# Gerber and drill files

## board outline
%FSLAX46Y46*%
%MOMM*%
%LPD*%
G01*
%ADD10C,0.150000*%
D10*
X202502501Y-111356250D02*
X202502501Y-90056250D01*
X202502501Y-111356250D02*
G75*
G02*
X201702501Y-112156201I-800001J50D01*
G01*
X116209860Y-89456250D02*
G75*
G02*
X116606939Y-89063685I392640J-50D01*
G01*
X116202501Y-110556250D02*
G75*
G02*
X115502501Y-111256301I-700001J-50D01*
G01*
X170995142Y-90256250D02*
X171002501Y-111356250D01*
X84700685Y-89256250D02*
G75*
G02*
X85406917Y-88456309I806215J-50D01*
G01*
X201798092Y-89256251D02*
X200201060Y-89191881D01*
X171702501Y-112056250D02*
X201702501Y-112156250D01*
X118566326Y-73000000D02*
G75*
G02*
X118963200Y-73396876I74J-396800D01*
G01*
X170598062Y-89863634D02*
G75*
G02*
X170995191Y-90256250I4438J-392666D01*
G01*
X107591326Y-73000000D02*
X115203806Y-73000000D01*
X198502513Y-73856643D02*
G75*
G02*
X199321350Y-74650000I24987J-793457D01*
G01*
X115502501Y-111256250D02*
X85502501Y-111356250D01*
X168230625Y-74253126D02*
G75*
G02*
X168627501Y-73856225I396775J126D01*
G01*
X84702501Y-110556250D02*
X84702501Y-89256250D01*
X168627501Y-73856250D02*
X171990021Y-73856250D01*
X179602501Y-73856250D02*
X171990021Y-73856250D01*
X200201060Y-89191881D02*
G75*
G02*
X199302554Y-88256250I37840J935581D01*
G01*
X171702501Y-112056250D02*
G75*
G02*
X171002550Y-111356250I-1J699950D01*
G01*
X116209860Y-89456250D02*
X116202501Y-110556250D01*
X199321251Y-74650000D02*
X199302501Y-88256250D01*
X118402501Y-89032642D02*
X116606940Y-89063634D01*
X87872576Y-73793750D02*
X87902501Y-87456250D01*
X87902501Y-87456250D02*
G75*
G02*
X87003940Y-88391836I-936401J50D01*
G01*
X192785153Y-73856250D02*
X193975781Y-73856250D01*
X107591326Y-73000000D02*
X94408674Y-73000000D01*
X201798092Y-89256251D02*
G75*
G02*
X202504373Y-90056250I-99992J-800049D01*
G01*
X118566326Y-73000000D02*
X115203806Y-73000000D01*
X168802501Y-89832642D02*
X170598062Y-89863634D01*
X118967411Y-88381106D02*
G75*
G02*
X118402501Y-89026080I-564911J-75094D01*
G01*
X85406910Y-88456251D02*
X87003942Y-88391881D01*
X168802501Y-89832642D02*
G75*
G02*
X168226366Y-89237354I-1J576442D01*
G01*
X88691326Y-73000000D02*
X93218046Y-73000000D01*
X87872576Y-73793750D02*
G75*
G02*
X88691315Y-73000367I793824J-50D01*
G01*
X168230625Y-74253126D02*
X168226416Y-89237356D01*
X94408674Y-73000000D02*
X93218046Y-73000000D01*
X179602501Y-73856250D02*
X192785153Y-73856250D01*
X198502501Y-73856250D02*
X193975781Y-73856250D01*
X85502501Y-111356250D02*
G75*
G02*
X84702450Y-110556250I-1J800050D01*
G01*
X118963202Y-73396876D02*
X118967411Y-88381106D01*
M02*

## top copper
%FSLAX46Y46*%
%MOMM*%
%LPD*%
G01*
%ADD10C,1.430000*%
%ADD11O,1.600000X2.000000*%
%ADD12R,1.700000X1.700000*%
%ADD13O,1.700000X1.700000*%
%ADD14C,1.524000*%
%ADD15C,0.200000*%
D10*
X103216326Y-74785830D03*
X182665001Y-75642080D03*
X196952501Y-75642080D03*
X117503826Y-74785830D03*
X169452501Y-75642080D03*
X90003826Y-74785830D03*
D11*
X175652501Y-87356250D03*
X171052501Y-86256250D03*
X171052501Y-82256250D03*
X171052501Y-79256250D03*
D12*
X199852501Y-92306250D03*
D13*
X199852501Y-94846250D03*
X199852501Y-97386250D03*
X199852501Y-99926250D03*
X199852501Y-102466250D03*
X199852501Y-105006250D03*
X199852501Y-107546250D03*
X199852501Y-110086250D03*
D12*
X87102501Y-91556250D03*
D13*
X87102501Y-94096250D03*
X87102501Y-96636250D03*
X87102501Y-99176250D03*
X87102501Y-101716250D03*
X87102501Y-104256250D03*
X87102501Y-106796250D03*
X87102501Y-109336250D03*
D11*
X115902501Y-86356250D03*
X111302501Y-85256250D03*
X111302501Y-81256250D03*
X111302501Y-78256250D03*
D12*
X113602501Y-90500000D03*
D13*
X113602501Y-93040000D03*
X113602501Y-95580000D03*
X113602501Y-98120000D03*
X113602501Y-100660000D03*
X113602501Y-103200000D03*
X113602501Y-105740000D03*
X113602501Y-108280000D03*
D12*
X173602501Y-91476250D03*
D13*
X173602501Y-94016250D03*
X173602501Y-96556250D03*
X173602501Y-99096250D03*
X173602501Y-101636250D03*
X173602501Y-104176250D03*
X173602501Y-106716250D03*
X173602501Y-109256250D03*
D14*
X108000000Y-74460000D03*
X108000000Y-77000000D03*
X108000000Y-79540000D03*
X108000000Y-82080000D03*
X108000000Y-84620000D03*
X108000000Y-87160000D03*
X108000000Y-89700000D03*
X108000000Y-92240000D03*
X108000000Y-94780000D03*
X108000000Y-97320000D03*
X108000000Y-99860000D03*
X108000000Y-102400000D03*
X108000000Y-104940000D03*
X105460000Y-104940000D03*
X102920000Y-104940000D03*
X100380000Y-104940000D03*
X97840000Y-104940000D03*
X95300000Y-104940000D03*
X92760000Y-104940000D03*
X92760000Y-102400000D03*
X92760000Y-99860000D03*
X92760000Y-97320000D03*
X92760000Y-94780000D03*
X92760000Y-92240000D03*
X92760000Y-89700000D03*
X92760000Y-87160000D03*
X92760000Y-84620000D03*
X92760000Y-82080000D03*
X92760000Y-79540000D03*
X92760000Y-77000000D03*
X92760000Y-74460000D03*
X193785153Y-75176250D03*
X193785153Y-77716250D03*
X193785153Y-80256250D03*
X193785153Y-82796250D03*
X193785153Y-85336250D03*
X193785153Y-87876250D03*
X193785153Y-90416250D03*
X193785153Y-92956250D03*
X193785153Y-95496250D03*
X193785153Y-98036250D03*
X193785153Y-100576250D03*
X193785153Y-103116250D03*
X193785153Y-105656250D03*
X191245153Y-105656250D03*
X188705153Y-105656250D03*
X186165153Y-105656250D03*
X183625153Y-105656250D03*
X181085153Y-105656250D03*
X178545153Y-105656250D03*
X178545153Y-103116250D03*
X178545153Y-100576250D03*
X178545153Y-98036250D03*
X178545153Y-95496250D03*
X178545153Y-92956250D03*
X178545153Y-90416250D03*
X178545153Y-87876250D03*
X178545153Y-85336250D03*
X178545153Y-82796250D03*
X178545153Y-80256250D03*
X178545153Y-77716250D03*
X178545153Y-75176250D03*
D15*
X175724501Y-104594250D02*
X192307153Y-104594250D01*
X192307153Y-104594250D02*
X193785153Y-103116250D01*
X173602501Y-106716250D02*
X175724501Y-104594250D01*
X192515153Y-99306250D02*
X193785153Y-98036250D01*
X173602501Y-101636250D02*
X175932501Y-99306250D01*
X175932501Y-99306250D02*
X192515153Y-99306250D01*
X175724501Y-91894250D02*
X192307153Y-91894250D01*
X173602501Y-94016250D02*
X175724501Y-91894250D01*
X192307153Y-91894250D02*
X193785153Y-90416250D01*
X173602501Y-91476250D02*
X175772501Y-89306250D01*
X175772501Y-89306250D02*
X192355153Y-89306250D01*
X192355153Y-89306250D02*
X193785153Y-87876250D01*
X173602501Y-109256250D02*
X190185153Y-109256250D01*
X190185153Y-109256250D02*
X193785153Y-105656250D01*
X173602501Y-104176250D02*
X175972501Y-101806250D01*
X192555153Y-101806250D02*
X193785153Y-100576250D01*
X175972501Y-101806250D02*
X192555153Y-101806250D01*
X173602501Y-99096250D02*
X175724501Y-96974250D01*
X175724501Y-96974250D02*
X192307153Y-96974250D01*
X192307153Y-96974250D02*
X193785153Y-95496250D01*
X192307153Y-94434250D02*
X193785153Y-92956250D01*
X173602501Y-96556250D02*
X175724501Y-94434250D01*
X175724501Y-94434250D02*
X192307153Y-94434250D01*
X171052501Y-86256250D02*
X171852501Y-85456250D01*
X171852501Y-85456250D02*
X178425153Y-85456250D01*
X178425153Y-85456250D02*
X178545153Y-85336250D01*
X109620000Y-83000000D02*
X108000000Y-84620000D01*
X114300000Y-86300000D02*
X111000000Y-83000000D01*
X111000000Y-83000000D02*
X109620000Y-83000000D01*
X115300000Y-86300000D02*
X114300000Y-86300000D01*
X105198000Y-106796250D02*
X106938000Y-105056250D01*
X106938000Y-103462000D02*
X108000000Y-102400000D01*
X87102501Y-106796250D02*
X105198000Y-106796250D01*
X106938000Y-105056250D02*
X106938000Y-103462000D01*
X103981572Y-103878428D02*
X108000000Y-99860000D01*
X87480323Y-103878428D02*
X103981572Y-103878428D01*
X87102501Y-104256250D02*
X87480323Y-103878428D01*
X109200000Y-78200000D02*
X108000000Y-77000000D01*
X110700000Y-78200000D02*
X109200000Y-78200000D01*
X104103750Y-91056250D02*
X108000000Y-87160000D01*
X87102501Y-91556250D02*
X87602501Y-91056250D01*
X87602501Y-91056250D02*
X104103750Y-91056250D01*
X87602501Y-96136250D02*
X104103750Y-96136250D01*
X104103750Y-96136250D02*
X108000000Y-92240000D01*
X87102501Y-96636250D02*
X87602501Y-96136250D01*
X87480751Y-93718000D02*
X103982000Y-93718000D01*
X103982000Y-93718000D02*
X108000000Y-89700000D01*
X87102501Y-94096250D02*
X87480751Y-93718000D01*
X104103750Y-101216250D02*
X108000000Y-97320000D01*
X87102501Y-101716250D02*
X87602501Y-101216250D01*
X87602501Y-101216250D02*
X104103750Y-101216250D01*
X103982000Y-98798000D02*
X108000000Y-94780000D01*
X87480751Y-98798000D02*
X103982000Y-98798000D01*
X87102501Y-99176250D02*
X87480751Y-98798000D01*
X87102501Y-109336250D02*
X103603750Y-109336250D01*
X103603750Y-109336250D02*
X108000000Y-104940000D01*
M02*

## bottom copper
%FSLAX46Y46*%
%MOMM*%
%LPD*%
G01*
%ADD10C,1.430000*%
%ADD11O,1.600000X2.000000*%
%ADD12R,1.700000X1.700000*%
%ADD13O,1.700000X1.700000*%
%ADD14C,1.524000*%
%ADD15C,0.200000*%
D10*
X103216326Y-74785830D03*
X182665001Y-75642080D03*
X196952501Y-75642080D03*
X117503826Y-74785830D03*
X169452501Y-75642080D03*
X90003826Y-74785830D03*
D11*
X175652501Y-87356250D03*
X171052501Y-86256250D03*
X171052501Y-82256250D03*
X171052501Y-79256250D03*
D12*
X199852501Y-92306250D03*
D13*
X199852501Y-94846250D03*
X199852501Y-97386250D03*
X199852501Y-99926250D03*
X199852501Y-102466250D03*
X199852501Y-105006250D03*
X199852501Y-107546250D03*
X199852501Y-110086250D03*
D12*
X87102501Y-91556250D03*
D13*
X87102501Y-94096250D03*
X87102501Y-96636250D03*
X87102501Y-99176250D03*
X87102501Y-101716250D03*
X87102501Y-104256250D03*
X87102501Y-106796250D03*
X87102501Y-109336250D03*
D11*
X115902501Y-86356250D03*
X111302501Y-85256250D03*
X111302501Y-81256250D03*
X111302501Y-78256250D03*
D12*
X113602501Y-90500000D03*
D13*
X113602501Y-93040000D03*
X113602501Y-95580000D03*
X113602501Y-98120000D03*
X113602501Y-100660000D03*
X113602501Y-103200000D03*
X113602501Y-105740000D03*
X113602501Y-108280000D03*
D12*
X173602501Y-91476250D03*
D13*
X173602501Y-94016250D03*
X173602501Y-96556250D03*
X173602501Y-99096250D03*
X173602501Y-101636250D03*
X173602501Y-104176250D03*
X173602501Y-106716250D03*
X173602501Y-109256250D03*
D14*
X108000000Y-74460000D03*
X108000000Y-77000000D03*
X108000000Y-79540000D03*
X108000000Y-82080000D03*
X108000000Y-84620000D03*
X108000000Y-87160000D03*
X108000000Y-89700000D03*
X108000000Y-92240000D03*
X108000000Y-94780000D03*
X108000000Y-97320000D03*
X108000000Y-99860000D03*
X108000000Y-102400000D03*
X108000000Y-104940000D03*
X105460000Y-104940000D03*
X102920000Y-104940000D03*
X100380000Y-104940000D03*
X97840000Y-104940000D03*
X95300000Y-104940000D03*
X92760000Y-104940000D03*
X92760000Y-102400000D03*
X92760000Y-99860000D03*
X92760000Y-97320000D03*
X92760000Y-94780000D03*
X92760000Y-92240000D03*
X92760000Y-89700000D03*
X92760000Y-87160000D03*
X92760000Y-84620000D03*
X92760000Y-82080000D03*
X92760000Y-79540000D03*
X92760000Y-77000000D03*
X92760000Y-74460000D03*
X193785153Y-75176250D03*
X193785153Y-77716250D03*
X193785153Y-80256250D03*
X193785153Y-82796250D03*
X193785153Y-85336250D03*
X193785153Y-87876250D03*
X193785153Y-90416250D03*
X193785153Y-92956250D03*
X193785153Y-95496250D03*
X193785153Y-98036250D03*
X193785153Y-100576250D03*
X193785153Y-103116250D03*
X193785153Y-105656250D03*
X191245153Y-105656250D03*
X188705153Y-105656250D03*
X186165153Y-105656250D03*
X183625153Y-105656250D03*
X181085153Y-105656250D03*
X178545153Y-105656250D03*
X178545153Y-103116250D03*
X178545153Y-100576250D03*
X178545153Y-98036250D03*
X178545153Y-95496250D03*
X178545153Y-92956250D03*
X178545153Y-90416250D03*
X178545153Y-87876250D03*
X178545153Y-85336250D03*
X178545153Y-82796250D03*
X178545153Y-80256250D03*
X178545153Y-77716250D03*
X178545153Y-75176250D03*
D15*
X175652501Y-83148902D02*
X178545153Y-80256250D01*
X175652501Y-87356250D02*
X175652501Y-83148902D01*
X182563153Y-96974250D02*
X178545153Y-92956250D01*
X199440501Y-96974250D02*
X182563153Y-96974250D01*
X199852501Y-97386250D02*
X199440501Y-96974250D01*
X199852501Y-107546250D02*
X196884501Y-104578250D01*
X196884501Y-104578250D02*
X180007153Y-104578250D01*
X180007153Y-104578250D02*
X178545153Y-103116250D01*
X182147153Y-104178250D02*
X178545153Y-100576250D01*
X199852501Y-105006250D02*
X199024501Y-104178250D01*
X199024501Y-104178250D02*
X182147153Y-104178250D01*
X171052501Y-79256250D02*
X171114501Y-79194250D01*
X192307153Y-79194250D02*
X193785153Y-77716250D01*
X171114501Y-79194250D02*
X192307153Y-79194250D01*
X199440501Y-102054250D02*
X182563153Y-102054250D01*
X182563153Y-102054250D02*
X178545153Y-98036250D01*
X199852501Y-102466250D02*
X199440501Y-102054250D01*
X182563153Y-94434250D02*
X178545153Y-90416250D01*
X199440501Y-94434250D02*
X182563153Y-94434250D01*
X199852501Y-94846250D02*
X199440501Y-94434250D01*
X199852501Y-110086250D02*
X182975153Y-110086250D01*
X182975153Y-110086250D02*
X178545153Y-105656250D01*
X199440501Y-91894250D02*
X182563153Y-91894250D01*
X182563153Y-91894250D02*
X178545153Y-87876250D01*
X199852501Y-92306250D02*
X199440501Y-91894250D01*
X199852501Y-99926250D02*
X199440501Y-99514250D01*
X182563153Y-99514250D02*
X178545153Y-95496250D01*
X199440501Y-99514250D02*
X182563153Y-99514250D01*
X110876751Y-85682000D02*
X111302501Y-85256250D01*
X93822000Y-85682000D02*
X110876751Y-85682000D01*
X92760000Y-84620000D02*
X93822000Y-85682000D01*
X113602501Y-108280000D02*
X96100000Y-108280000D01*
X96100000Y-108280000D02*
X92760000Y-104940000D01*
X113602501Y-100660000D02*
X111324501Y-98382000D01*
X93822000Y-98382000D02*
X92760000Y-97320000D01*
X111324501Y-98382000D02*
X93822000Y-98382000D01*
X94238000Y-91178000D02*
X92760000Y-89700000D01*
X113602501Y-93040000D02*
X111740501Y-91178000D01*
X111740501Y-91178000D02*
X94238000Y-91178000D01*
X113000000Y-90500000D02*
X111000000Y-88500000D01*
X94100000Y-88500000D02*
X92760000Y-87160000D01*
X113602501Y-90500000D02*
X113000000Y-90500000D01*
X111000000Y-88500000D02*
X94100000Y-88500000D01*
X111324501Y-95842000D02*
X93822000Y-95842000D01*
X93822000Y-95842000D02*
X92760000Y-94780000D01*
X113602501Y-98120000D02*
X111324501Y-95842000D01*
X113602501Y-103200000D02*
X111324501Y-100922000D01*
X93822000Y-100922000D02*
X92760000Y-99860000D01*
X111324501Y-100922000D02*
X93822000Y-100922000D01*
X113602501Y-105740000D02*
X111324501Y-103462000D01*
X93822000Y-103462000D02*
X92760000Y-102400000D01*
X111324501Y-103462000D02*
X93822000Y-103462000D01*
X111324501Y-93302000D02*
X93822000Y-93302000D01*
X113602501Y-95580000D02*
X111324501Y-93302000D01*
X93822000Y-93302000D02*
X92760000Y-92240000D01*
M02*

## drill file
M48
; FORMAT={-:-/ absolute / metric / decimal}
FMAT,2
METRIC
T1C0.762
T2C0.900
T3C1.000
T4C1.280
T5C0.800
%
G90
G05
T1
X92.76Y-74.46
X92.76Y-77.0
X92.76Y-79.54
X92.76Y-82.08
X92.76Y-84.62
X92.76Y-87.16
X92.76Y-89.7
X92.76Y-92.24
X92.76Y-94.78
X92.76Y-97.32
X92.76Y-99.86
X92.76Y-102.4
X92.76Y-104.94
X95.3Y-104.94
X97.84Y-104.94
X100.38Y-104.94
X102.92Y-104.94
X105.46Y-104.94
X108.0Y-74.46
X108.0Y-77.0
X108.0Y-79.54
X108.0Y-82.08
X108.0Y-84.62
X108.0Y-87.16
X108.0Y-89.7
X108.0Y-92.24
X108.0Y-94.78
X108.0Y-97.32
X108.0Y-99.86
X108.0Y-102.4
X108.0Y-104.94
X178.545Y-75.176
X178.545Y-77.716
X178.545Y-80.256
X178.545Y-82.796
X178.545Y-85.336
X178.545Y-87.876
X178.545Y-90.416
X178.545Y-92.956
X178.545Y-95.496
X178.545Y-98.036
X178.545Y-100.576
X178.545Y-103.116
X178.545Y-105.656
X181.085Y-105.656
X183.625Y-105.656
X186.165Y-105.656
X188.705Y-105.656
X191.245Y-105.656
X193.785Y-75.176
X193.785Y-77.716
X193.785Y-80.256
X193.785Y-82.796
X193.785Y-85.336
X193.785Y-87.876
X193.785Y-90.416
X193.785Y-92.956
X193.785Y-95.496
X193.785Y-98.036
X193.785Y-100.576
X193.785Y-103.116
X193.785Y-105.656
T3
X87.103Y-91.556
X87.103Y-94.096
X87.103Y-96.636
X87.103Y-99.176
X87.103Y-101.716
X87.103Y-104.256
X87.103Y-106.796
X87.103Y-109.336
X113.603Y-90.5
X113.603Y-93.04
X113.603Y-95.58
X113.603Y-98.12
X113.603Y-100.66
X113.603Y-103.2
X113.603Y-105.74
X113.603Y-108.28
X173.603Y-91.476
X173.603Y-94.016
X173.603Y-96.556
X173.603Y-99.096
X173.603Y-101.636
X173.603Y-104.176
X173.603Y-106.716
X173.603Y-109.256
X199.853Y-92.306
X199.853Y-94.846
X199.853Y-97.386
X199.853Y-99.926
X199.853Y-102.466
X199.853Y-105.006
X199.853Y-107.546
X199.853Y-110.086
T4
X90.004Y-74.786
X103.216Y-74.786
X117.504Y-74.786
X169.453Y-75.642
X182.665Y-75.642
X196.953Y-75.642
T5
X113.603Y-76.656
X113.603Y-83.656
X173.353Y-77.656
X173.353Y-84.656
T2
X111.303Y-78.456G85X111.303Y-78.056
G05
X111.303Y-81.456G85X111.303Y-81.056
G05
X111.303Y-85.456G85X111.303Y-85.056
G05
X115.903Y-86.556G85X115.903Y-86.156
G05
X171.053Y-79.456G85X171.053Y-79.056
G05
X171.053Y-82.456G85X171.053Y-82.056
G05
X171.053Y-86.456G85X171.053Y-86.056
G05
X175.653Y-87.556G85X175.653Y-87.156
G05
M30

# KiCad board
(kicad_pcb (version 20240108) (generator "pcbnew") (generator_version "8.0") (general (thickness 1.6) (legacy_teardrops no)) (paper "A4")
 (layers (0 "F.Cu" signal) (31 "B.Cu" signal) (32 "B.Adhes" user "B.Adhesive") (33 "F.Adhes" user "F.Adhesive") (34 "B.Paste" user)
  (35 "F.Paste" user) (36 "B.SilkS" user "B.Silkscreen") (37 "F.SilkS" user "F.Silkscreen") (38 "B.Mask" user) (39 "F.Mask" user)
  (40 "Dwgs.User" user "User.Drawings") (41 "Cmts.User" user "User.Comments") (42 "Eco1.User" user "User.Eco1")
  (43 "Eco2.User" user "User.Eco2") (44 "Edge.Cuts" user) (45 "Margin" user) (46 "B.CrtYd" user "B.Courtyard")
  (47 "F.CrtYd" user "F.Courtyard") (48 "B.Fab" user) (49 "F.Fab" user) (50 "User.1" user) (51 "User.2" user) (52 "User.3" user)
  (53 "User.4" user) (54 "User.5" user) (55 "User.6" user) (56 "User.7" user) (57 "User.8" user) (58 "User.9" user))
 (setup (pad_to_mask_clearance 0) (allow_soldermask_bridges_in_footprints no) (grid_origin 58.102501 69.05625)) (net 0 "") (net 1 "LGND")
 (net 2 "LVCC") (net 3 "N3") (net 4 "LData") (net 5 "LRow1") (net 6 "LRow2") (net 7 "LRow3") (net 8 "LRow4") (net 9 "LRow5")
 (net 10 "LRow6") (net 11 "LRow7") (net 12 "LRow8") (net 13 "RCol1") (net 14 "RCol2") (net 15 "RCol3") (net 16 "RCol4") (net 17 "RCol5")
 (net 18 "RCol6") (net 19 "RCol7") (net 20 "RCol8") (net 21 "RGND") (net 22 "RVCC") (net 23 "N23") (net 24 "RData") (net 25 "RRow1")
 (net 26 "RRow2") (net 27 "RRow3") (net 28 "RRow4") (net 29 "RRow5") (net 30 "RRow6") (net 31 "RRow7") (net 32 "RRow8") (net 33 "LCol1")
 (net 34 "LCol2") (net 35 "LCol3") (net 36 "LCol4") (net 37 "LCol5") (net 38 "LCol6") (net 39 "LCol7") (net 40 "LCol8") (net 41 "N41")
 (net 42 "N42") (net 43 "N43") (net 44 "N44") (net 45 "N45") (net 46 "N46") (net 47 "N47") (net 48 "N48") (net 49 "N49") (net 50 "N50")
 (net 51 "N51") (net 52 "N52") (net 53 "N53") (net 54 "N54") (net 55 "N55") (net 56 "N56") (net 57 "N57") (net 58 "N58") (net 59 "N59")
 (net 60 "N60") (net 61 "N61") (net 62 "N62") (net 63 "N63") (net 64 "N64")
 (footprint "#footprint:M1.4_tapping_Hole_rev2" (layer "F.Cu") (at 103.216326 74.78583 -90)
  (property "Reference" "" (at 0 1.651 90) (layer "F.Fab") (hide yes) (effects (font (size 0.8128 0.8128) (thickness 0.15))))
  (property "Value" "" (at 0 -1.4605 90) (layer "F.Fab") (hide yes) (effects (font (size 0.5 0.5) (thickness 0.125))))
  (pad "" thru_hole circle (at 0 0 270) (size 1.43 1.43) (drill 1.28) (layers "*.Cu" "*.Mask") (remove_unused_layers no)))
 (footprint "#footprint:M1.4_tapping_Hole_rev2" (layer "F.Cu") (at 182.665001 75.64208 -90)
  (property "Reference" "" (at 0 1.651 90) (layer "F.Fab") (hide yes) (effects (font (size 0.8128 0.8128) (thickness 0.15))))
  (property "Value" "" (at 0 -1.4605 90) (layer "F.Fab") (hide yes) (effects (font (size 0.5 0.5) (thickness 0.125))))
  (pad "" thru_hole circle (at 0 0 270) (size 1.43 1.43) (drill 1.28) (layers "*.Cu" "*.Mask") (remove_unused_layers no)))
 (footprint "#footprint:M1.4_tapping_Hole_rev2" (layer "F.Cu") (at 196.952501 75.64208 -90)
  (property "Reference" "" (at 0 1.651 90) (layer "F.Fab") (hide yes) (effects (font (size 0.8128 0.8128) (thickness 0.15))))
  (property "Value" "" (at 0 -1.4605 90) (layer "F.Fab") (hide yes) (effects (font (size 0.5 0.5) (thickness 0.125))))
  (pad "" thru_hole circle (at 0 0 270) (size 1.43 1.43) (drill 1.28) (layers "*.Cu" "*.Mask") (remove_unused_layers no)))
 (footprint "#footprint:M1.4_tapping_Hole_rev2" (layer "F.Cu") (at 117.503826 74.78583 -90)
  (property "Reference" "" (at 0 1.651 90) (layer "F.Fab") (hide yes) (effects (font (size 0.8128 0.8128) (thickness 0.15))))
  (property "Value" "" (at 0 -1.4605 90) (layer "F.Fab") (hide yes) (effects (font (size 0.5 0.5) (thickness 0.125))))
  (pad "" thru_hole circle (at 0 0 270) (size 1.43 1.43) (drill 1.28) (layers "*.Cu" "*.Mask") (remove_unused_layers no)))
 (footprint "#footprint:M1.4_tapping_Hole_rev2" (layer "F.Cu") (at 169.452501 75.044581 -90)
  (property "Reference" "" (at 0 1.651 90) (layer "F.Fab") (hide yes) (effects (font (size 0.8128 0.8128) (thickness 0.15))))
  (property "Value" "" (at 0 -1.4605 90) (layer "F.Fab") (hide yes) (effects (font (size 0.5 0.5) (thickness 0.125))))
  (pad "" thru_hole circle (at 0.597499 0 270) (size 1.43 1.43) (drill 1.28) (layers "*.Cu" "*.Mask") (remove_unused_layers no)))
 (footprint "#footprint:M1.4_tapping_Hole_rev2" (layer "F.Cu") (at 90.003826 74.188331 -90)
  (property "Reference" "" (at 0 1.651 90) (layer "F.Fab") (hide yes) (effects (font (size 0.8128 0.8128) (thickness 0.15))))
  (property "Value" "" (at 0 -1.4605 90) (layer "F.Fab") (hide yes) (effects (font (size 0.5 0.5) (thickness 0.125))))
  (pad "" thru_hole circle (at 0.597499 0 270) (size 1.43 1.43) (drill 1.28) (layers "*.Cu" "*.Mask") (remove_unused_layers no)))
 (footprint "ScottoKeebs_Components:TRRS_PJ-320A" (layer "B.Cu") (at 173.352501 76.05625 180)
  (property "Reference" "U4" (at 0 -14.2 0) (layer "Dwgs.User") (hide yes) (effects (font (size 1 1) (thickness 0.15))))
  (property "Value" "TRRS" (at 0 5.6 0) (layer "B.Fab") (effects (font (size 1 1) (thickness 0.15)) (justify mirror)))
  (pad "" np_thru_hole circle (at 0 -8.6 180) (size 0.8 0.8) (drill 0.8) (layers "*.Cu" "*.Mask"))
  (pad "" np_thru_hole circle (at 0 -1.6 180) (size 0.8 0.8) (drill 0.8) (layers "*.Cu" "*.Mask"))
  (pad "1" thru_hole oval (at -2.3 -11.3 180) (size 1.6 2) (drill oval 0.9 1.3) (layers "*.Cu" "*.Mask") (remove_unused_layers no)
   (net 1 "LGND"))
  (pad "2" thru_hole oval (at 2.3 -10.2 180) (size 1.6 2) (drill oval 0.9 1.3) (layers "*.Cu" "*.Mask") (remove_unused_layers no)
   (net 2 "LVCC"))
  (pad "3" thru_hole oval (at 2.3 -6.2 180) (size 1.6 2) (drill oval 0.9 1.3) (layers "*.Cu" "*.Mask") (remove_unused_layers no)
   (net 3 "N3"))
  (pad "4" thru_hole oval (at 2.3 -3.2 180) (size 1.6 2) (drill oval 0.9 1.3) (layers "*.Cu" "*.Mask") (remove_unused_layers no)
   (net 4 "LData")))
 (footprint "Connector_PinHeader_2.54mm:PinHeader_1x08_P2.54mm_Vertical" (layer "B.Cu") (at 199.852501 92.30625 180)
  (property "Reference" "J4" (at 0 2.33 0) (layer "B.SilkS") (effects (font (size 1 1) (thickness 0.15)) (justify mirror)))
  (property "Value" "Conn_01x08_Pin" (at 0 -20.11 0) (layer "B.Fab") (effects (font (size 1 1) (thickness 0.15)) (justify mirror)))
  (pad "1" thru_hole rect (at 0 0 180) (size 1.7 1.7) (drill 1) (layers "*.Cu" "*.Mask") (remove_unused_layers no) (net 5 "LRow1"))
  (pad "2" thru_hole oval (at 0 -2.54 180) (size 1.7 1.7) (drill 1) (layers "*.Cu" "*.Mask") (remove_unused_layers no) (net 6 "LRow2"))
  (pad "3" thru_hole oval (at 0 -5.08 180) (size 1.7 1.7) (drill 1) (layers "*.Cu" "*.Mask") (remove_unused_layers no) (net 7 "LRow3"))
  (pad "4" thru_hole oval (at 0 -7.62 180) (size 1.7 1.7) (drill 1) (layers "*.Cu" "*.Mask") (remove_unused_layers no) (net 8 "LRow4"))
  (pad "5" thru_hole oval (at 0 -10.16 180) (size 1.7 1.7) (drill 1) (layers "*.Cu" "*.Mask") (remove_unused_layers no) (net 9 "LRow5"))
  (pad "6" thru_hole oval (at 0 -12.7 180) (size 1.7 1.7) (drill 1) (layers "*.Cu" "*.Mask") (remove_unused_layers no) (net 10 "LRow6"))
  (pad "7" thru_hole oval (at 0 -15.24 180) (size 1.7 1.7) (drill 1) (layers "*.Cu" "*.Mask") (remove_unused_layers no) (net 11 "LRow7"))
  (pad "8" thru_hole oval (at 0 -17.78 180) (size 1.7 1.7) (drill 1) (layers "*.Cu" "*.Mask") (remove_unused_layers no) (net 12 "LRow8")))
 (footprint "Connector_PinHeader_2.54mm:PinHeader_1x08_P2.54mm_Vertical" (layer "B.Cu") (at 87.102501 91.55625 180)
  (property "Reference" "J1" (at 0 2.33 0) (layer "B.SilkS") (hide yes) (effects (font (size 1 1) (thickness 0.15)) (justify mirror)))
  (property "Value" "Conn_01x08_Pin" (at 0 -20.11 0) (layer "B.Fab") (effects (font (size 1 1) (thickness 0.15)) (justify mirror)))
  (pad "1" thru_hole rect (at 0 0 180) (size 1.7 1.7) (drill 1) (layers "*.Cu" "*.Mask") (remove_unused_layers no) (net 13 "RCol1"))
  (pad "2" thru_hole oval (at 0 -2.54 180) (size 1.7 1.7) (drill 1) (layers "*.Cu" "*.Mask") (remove_unused_layers no) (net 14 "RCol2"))
  (pad "3" thru_hole oval (at 0 -5.08 180) (size 1.7 1.7) (drill 1) (layers "*.Cu" "*.Mask") (remove_unused_layers no) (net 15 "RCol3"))
  (pad "4" thru_hole oval (at 0 -7.62 180) (size 1.7 1.7) (drill 1) (layers "*.Cu" "*.Mask") (remove_unused_layers no) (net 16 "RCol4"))
  (pad "5" thru_hole oval (at 0 -10.16 180) (size 1.7 1.7) (drill 1) (layers "*.Cu" "*.Mask") (remove_unused_layers no) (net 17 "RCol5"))
  (pad "6" thru_hole oval (at 0 -12.7 180) (size 1.7 1.7) (drill 1) (layers "*.Cu" "*.Mask") (remove_unused_layers no) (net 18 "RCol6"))
  (pad "7" thru_hole oval (at 0 -15.24 180) (size 1.7 1.7) (drill 1) (layers "*.Cu" "*.Mask") (remove_unused_layers no) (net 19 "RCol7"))
  (pad "8" thru_hole oval (at 0 -17.78 180) (size 1.7 1.7) (drill 1) (layers "*.Cu" "*.Mask") (remove_unused_layers no) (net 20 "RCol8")))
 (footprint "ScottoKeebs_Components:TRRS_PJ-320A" (layer "B.Cu") (at 113.602501 75.05625 180)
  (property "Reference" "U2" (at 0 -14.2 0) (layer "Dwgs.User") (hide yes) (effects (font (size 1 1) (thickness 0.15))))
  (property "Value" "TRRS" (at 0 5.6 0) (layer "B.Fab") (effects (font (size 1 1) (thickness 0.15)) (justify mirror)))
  (pad "" np_thru_hole circle (at 0 -8.6 180) (size 0.8 0.8) (drill 0.8) (layers "*.Cu" "*.Mask"))
  (pad "" np_thru_hole circle (at 0 -1.6 180) (size 0.8 0.8) (drill 0.8) (layers "*.Cu" "*.Mask"))
  (pad "1" thru_hole oval (at -2.3 -11.3 180) (size 1.6 2) (drill oval 0.9 1.3) (layers "*.Cu" "*.Mask") (remove_unused_layers no)
   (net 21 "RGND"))
  (pad "2" thru_hole oval (at 2.3 -10.2 180) (size 1.6 2) (drill oval 0.9 1.3) (layers "*.Cu" "*.Mask") (remove_unused_layers no)
   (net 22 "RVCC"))
  (pad "3" thru_hole oval (at 2.3 -6.2 180) (size 1.6 2) (drill oval 0.9 1.3) (layers "*.Cu" "*.Mask") (remove_unused_layers no)
   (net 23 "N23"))
  (pad "4" thru_hole oval (at 2.3 -3.2 180) (size 1.6 2) (drill oval 0.9 1.3) (layers "*.Cu" "*.Mask") (remove_unused_layers no)
   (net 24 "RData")))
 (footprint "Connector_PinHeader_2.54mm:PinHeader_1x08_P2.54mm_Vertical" (layer "B.Cu") (at 113.602501 90.5 180)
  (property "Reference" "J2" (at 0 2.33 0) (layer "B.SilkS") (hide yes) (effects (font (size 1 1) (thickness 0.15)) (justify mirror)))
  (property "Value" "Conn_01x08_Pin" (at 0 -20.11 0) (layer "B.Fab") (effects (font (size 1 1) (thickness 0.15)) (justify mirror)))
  (pad "1" thru_hole rect (at 0 0 180) (size 1.7 1.7) (drill 1) (layers "*.Cu" "*.Mask") (remove_unused_layers no) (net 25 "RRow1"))
  (pad "2" thru_hole oval (at 0 -2.54 180) (size 1.7 1.7) (drill 1) (layers "*.Cu" "*.Mask") (remove_unused_layers no) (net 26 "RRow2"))
  (pad "3" thru_hole oval (at 0 -5.08 180) (size 1.7 1.7) (drill 1) (layers "*.Cu" "*.Mask") (remove_unused_layers no) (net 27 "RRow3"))
  (pad "4" thru_hole oval (at 0 -7.62 180) (size 1.7 1.7) (drill 1) (layers "*.Cu" "*.Mask") (remove_unused_layers no) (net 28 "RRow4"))
  (pad "5" thru_hole oval (at 0 -10.16 180) (size 1.7 1.7) (drill 1) (layers "*.Cu" "*.Mask") (remove_unused_layers no) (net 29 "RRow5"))
  (pad "6" thru_hole oval (at 0 -12.7 180) (size 1.7 1.7) (drill 1) (layers "*.Cu" "*.Mask") (remove_unused_layers no) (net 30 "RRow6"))
  (pad "7" thru_hole oval (at 0 -15.24 180) (size 1.7 1.7) (drill 1) (layers "*.Cu" "*.Mask") (remove_unused_layers no) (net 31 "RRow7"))
  (pad "8" thru_hole oval (at 0 -17.78 180) (size 1.7 1.7) (drill 1) (layers "*.Cu" "*.Mask") (remove_unused_layers no) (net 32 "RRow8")))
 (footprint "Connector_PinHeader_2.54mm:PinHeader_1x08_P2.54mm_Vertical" (layer "B.Cu") (at 173.602501 91.47625 180)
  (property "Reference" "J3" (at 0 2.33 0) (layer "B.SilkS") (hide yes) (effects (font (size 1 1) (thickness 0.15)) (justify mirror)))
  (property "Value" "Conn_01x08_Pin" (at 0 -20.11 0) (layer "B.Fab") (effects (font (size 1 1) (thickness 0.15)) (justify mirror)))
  (pad "1" thru_hole rect (at 0 0 180) (size 1.7 1.7) (drill 1) (layers "*.Cu" "*.Mask") (remove_unused_layers no) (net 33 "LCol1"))
  (pad "2" thru_hole oval (at 0 -2.54 180) (size 1.7 1.7) (drill 1) (layers "*.Cu" "*.Mask") (remove_unused_layers no) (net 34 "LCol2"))
  (pad "3" thru_hole oval (at 0 -5.08 180) (size 1.7 1.7) (drill 1) (layers "*.Cu" "*.Mask") (remove_unused_layers no) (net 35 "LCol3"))
  (pad "4" thru_hole oval (at 0 -7.62 180) (size 1.7 1.7) (drill 1) (layers "*.Cu" "*.Mask") (remove_unused_layers no) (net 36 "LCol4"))
  (pad "5" thru_hole oval (at 0 -10.16 180) (size 1.7 1.7) (drill 1) (layers "*.Cu" "*.Mask") (remove_unused_layers no) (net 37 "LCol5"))
  (pad "6" thru_hole oval (at 0 -12.7 180) (size 1.7 1.7) (drill 1) (layers "*.Cu" "*.Mask") (remove_unused_layers no) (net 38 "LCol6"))
  (pad "7" thru_hole oval (at 0 -15.24 180) (size 1.7 1.7) (drill 1) (layers "*.Cu" "*.Mask") (remove_unused_layers no) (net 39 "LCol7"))
  (pad "8" thru_hole oval (at 0 -17.78 180) (size 1.7 1.7) (drill 1) (layers "*.Cu" "*.Mask") (remove_unused_layers no) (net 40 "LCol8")))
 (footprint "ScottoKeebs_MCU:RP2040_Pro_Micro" (layer "B.Cu") (at 100.38 90.97 180)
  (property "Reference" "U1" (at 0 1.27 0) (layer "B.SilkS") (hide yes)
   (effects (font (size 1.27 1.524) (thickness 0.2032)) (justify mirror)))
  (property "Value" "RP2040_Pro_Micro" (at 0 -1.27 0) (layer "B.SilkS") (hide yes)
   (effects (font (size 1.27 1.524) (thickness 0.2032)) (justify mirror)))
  (pad "1" thru_hole circle (at -7.62 16.51 180) (size 1.524 1.524) (drill 0.762) (layers "*.Cu" "*.Mask") (remove_unused_layers no)
   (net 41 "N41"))
  (pad "2" thru_hole circle (at -7.62 13.97 180) (size 1.524 1.524) (drill 0.762) (layers "*.Cu" "*.Mask") (remove_unused_layers no)
   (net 24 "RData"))
  (pad "3" thru_hole circle (at -7.62 11.43 180) (size 1.524 1.524) (drill 0.762) (layers "*.Cu" "*.Mask") (remove_unused_layers no)
   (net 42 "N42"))
  (pad "4" thru_hole circle (at -7.62 8.89 180) (size 1.524 1.524) (drill 0.762) (layers "*.Cu" "*.Mask") (remove_unused_layers no)
   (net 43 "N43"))
  (pad "5" thru_hole circle (at -7.62 6.35 180) (size 1.524 1.524) (drill 0.762) (layers "*.Cu" "*.Mask") (remove_unused_layers no)
   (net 21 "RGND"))
  (pad "6" thru_hole circle (at -7.62 3.81 180) (size 1.524 1.524) (drill 0.762) (layers "*.Cu" "*.Mask") (remove_unused_layers no)
   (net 13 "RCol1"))
  (pad "7" thru_hole circle (at -7.62 1.27 180) (size 1.524 1.524) (drill 0.762) (layers "*.Cu" "*.Mask") (remove_unused_layers no)
   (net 14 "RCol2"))
  (pad "8" thru_hole circle (at -7.62 -1.27 180) (size 1.524 1.524) (drill 0.762) (layers "*.Cu" "*.Mask") (remove_unused_layers no)
   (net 15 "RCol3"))
  (pad "9" thru_hole circle (at -7.62 -3.81 180) (size 1.524 1.524) (drill 0.762) (layers "*.Cu" "*.Mask") (remove_unused_layers no)
   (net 16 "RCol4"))
  (pad "10" thru_hole circle (at -7.62 -6.35 180) (size 1.524 1.524) (drill 0.762) (layers "*.Cu" "*.Mask") (remove_unused_layers no)
   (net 17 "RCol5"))
  (pad "11" thru_hole circle (at -7.62 -8.89 180) (size 1.524 1.524) (drill 0.762) (layers "*.Cu" "*.Mask") (remove_unused_layers no)
   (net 18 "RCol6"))
  (pad "12" thru_hole circle (at -7.62 -11.43 180) (size 1.524 1.524) (drill 0.762) (layers "*.Cu" "*.Mask") (remove_unused_layers no)
   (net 19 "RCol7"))
  (pad "13" thru_hole circle (at -7.62 -13.97 180) (size 1.524 1.524) (drill 0.762) (layers "*.Cu" "*.Mask") (remove_unused_layers no)
   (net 20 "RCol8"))
  (pad "14" thru_hole circle (at -5.08 -13.97 180) (size 1.524 1.524) (drill 0.762) (layers "*.Cu" "*.Mask") (remove_unused_layers no)
   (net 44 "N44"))
  (pad "15" thru_hole circle (at -2.54 -13.97 180) (size 1.524 1.524) (drill 0.762) (layers "*.Cu" "*.Mask") (remove_unused_layers no)
   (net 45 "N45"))
  (pad "16" thru_hole circle (at 0 -13.97 180) (size 1.524 1.524) (drill 0.762) (layers "*.Cu" "*.Mask") (remove_unused_layers no)
   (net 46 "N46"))
  (pad "17" thru_hole circle (at 2.54 -13.97 180) (size 1.524 1.524) (drill 0.762) (layers "*.Cu" "*.Mask") (remove_unused_layers no)
   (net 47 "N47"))
  (pad "18" thru_hole circle (at 5.08 -13.97 180) (size 1.524 1.524) (drill 0.762) (layers "*.Cu" "*.Mask") (remove_unused_layers no)
   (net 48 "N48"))
  (pad "19" thru_hole circle (at 7.62 -13.97 180) (size 1.524 1.524) (drill 0.762) (layers "*.Cu" "*.Mask") (remove_unused_layers no)
   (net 32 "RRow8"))
  (pad "20" thru_hole circle (at 7.62 -11.43 180) (size 1.524 1.524) (drill 0.762) (layers "*.Cu" "*.Mask") (remove_unused_layers no)
   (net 31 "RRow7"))
  (pad "21" thru_hole circle (at 7.62 -8.89 180) (size 1.524 1.524) (drill 0.762) (layers "*.Cu" "*.Mask") (remove_unused_layers no)
   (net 30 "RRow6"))
  (pad "22" thru_hole circle (at 7.62 -6.35 180) (size 1.524 1.524) (drill 0.762) (layers "*.Cu" "*.Mask") (remove_unused_layers no)
   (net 29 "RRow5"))
  (pad "23" thru_hole circle (at 7.62 -3.81 180) (size 1.524 1.524) (drill 0.762) (layers "*.Cu" "*.Mask") (remove_unused_layers no)
   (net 28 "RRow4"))
  (pad "24" thru_hole circle (at 7.62 -1.27 180) (size 1.524 1.524) (drill 0.762) (layers "*.Cu" "*.Mask") (remove_unused_layers no)
   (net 27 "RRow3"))
  (pad "25" thru_hole circle (at 7.62 1.27 180) (size 1.524 1.524) (drill 0.762) (layers "*.Cu" "*.Mask") (remove_unused_layers no)
   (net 26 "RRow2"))
  (pad "26" thru_hole circle (at 7.62 3.81 180) (size 1.524 1.524) (drill 0.762) (layers "*.Cu" "*.Mask") (remove_unused_layers no)
   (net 25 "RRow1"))
  (pad "27" thru_hole circle (at 7.62 6.35 180) (size 1.524 1.524) (drill 0.762) (layers "*.Cu" "*.Mask") (remove_unused_layers no)
   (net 22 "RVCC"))
  (pad "28" thru_hole circle (at 7.62 8.89 180) (size 1.524 1.524) (drill 0.762) (layers "*.Cu" "*.Mask") (remove_unused_layers no)
   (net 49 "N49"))
  (pad "29" thru_hole circle (at 7.62 11.43 180) (size 1.524 1.524) (drill 0.762) (layers "*.Cu" "*.Mask") (remove_unused_layers no)
   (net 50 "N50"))
  (pad "30" thru_hole circle (at 7.62 13.97 180) (size 1.524 1.524) (drill 0.762) (layers "*.Cu" "*.Mask") (remove_unused_layers no)
   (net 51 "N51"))
  (pad "31" thru_hole circle (at 7.62 16.51 180) (size 1.524 1.524) (drill 0.762) (layers "*.Cu" "*.Mask") (remove_unused_layers no)
   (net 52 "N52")))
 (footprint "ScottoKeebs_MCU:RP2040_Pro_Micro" (layer "B.Cu") (at 186.165153 91.68625 180)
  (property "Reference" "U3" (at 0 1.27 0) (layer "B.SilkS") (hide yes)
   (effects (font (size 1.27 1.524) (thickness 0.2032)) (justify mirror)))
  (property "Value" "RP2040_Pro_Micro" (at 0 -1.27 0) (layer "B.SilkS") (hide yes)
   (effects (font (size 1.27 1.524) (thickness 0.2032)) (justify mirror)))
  (pad "1" thru_hole circle (at -7.62 16.51 180) (size 1.524 1.524) (drill 0.762) (layers "*.Cu" "*.Mask") (remove_unused_layers no)
   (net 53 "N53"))
  (pad "2" thru_hole circle (at -7.62 13.97 180) (size 1.524 1.524) (drill 0.762) (layers "*.Cu" "*.Mask") (remove_unused_layers no)
   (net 4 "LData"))
  (pad "3" thru_hole circle (at -7.62 11.43 180) (size 1.524 1.524) (drill 0.762) (layers "*.Cu" "*.Mask") (remove_unused_layers no)
   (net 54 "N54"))
  (pad "4" thru_hole circle (at -7.62 8.89 180) (size 1.524 1.524) (drill 0.762) (layers "*.Cu" "*.Mask") (remove_unused_layers no)
   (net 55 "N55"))
  (pad "5" thru_hole circle (at -7.62 6.35 180) (size 1.524 1.524) (drill 0.762) (layers "*.Cu" "*.Mask") (remove_unused_layers no)
   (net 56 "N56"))
  (pad "6" thru_hole circle (at -7.62 3.81 180) (size 1.524 1.524) (drill 0.762) (layers "*.Cu" "*.Mask") (remove_unused_layers no)
   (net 33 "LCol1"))
  (pad "7" thru_hole circle (at -7.62 1.27 180) (size 1.524 1.524) (drill 0.762) (layers "*.Cu" "*.Mask") (remove_unused_layers no)
   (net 34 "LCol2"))
  (pad "8" thru_hole circle (at -7.62 -1.27 180) (size 1.524 1.524) (drill 0.762) (layers "*.Cu" "*.Mask") (remove_unused_layers no)
   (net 35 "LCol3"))
  (pad "9" thru_hole circle (at -7.62 -3.81 180) (size 1.524 1.524) (drill 0.762) (layers "*.Cu" "*.Mask") (remove_unused_layers no)
   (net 36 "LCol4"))
  (pad "10" thru_hole circle (at -7.62 -6.35 180) (size 1.524 1.524) (drill 0.762) (layers "*.Cu" "*.Mask") (remove_unused_layers no)
   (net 37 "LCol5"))
  (pad "11" thru_hole circle (at -7.62 -8.89 180) (size 1.524 1.524) (drill 0.762) (layers "*.Cu" "*.Mask") (remove_unused_layers no)
   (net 38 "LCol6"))
  (pad "12" thru_hole circle (at -7.62 -11.43 180) (size 1.524 1.524) (drill 0.762) (layers "*.Cu" "*.Mask") (remove_unused_layers no)
   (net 39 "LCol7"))
  (pad "13" thru_hole circle (at -7.62 -13.97 180) (size 1.524 1.524) (drill 0.762) (layers "*.Cu" "*.Mask") (remove_unused_layers no)
   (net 40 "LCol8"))
  (pad "14" thru_hole circle (at -5.08 -13.97 180) (size 1.524 1.524) (drill 0.762) (layers "*.Cu" "*.Mask") (remove_unused_layers no)
   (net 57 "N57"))
  (pad "15" thru_hole circle (at -2.54 -13.97 180) (size 1.524 1.524) (drill 0.762) (layers "*.Cu" "*.Mask") (remove_unused_layers no)
   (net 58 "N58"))
  (pad "16" thru_hole circle (at 0 -13.97 180) (size 1.524 1.524) (drill 0.762) (layers "*.Cu" "*.Mask") (remove_unused_layers no)
   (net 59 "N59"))
  (pad "17" thru_hole circle (at 2.54 -13.97 180) (size 1.524 1.524) (drill 0.762) (layers "*.Cu" "*.Mask") (remove_unused_layers no)
   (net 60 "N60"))
  (pad "18" thru_hole circle (at 5.08 -13.97 180) (size 1.524 1.524) (drill 0.762) (layers "*.Cu" "*.Mask") (remove_unused_layers no)
   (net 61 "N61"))
  (pad "19" thru_hole circle (at 7.62 -13.97 180) (size 1.524 1.524) (drill 0.762) (layers "*.Cu" "*.Mask") (remove_unused_layers no)
   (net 12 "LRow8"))
  (pad "20" thru_hole circle (at 7.62 -11.43 180) (size 1.524 1.524) (drill 0.762) (layers "*.Cu" "*.Mask") (remove_unused_layers no)
   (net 11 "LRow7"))
  (pad "21" thru_hole circle (at 7.62 -8.89 180) (size 1.524 1.524) (drill 0.762) (layers "*.Cu" "*.Mask") (remove_unused_layers no)
   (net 10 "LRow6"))
  (pad "22" thru_hole circle (at 7.62 -6.35 180) (size 1.524 1.524) (drill 0.762) (layers "*.Cu" "*.Mask") (remove_unused_layers no)
   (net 9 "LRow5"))
  (pad "23" thru_hole circle (at 7.62 -3.81 180) (size 1.524 1.524) (drill 0.762) (layers "*.Cu" "*.Mask") (remove_unused_layers no)
   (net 8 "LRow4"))
  (pad "24" thru_hole circle (at 7.62 -1.27 180) (size 1.524 1.524) (drill 0.762) (layers "*.Cu" "*.Mask") (remove_unused_layers no)
   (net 7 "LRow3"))
  (pad "25" thru_hole circle (at 7.62 1.27 180) (size 1.524 1.524) (drill 0.762) (layers "*.Cu" "*.Mask") (remove_unused_layers no)
   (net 6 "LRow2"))
  (pad "26" thru_hole circle (at 7.62 3.81 180) (size 1.524 1.524) (drill 0.762) (layers "*.Cu" "*.Mask") (remove_unused_layers no)
   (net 5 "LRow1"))
  (pad "27" thru_hole circle (at 7.62 6.35 180) (size 1.524 1.524) (drill 0.762) (layers "*.Cu" "*.Mask") (remove_unused_layers no)
   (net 2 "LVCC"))
  (pad "28" thru_hole circle (at 7.62 8.89 180) (size 1.524 1.524) (drill 0.762) (layers "*.Cu" "*.Mask") (remove_unused_layers no)
   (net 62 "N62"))
  (pad "29" thru_hole circle (at 7.62 11.43 180) (size 1.524 1.524) (drill 0.762) (layers "*.Cu" "*.Mask") (remove_unused_layers no)
   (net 1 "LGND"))
  (pad "30" thru_hole circle (at 7.62 13.97 180) (size 1.524 1.524) (drill 0.762) (layers "*.Cu" "*.Mask") (remove_unused_layers no)
   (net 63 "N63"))
  (pad "31" thru_hole circle (at 7.62 16.51 180) (size 1.524 1.524) (drill 0.762) (layers "*.Cu" "*.Mask") (remove_unused_layers no)
   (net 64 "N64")))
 (gr_line (start 202.502501 111.35625) (end 202.502501 90.05625) (stroke (width 0.15) (type default)) (layer "Edge.Cuts"))
 (gr_arc (start 202.502501 111.35625) (mid 202.268186 111.921935) (end 201.702501 112.15625) (stroke (width 0.15) (type default))
  (layer "Edge.Cuts"))
 (gr_arc (start 116.20986 89.45625) (mid 116.326436 89.177046) (end 116.60694 89.063634) (stroke (width 0.15) (type default))
  (layer "Edge.Cuts"))
 (gr_arc (start 116.202501 110.55625) (mid 115.997476 111.051225) (end 115.502501 111.25625) (stroke (width 0.15) (type default))
  (layer "Edge.Cuts"))
 (gr_line (start 170.995142 90.25625) (end 171.002501 111.35625) (stroke (width 0.15) (type default)) (layer "Edge.Cuts"))
 (gr_arc (start 84.700685 89.25625) (mid 84.902501 88.722691) (end 85.40691 88.456251) (stroke (width 0.15) (type default))
  (layer "Edge.Cuts"))
 (gr_line (start 201.798092 89.256251) (end 200.20106 89.191881) (stroke (width 0.15) (type default)) (layer "Edge.Cuts"))
 (gr_line (start 171.702501 112.05625) (end 201.702501 112.15625) (stroke (width 0.15) (type default)) (layer "Edge.Cuts"))
 (gr_arc (start 118.566326 73) (mid 118.846973 73.116229) (end 118.963202 73.396876) (stroke (width 0.15) (type solid)) (layer "Edge.Cuts"))
 (gr_arc (start 170.598062 89.863634) (mid 170.878566 89.977046) (end 170.995142 90.25625) (stroke (width 0.15) (type default))
  (layer "Edge.Cuts"))
 (gr_line (start 107.591326 73) (end 115.203806 73) (stroke (width 0.15) (type solid)) (layer "Edge.Cuts"))
 (gr_arc (start 198.502513 73.856643) (mid 199.079847 74.079983) (end 199.321251 74.65) (stroke (width 0.15) (type solid))
  (layer "Edge.Cuts"))
 (gr_line (start 115.502501 111.25625) (end 85.502501 111.35625) (stroke (width 0.15) (type default)) (layer "Edge.Cuts"))
 (gr_arc (start 168.230625 74.253126) (mid 168.346843 73.97246) (end 168.627501 73.85625) (stroke (width 0.15) (type solid))
  (layer "Edge.Cuts"))
 (gr_line (start 84.702501 110.55625) (end 84.702501 89.25625) (stroke (width 0.15) (type default)) (layer "Edge.Cuts"))
 (gr_line (start 168.627501 73.85625) (end 171.990021 73.85625) (stroke (width 0.15) (type solid)) (layer "Edge.Cuts"))
 (gr_line (start 179.602501 73.85625) (end 171.990021 73.85625) (stroke (width 0.15) (type solid)) (layer "Edge.Cuts"))
 (gr_arc (start 200.20106 89.191881) (mid 199.563519 88.904867) (end 199.302501 88.25625) (stroke (width 0.15) (type default))
  (layer "Edge.Cuts"))
 (gr_arc (start 171.702501 112.05625) (mid 171.207526 111.851225) (end 171.002501 111.35625) (stroke (width 0.15) (type default))
  (layer "Edge.Cuts"))
 (gr_line (start 116.20986 89.45625) (end 116.202501 110.55625) (stroke (width 0.15) (type default)) (layer "Edge.Cuts"))
 (gr_line (start 199.321251 74.65) (end 199.302501 88.25625) (stroke (width 0.15) (type default)) (layer "Edge.Cuts"))
 (gr_line (start 118.402501 89.032642) (end 116.60694 89.063634) (stroke (width 0.15) (type default)) (layer "Edge.Cuts"))
 (gr_line (start 87.872576 73.79375) (end 87.902501 87.45625) (stroke (width 0.15) (type default)) (layer "Edge.Cuts"))
 (gr_arc (start 87.902501 87.45625) (mid 87.641481 88.104865) (end 87.003942 88.391881) (stroke (width 0.15) (type default))
  (layer "Edge.Cuts"))
 (gr_line (start 192.785153 73.85625) (end 193.975781 73.85625) (stroke (width 0.15) (type solid)) (layer "Edge.Cuts"))
 (gr_line (start 107.591326 73) (end 94.408674 73) (stroke (width 0.15) (type solid)) (layer "Edge.Cuts"))
 (gr_arc (start 201.798092 89.256251) (mid 202.302501 89.522688) (end 202.504317 90.05625) (stroke (width 0.15) (type default))
  (layer "Edge.Cuts"))
 (gr_line (start 118.566326 73) (end 115.203806 73) (stroke (width 0.15) (type solid)) (layer "Edge.Cuts"))
 (gr_line (start 168.802501 89.832642) (end 170.598062 89.863634) (stroke (width 0.15) (type default)) (layer "Edge.Cuts"))
 (gr_arc (start 118.967411 88.381106) (mid 118.831195 88.831679) (end 118.402501 89.02608) (stroke (width 0.15) (type default))
  (layer "Edge.Cuts"))
 (gr_line (start 85.40691 88.456251) (end 87.003942 88.391881) (stroke (width 0.15) (type default)) (layer "Edge.Cuts"))
 (gr_arc (start 168.802501 89.832642) (mid 168.388303 89.657085) (end 168.226417 89.237356) (stroke (width 0.15) (type default))
  (layer "Edge.Cuts"))
 (gr_line (start 88.691326 73) (end 93.218046 73) (stroke (width 0.15) (type solid)) (layer "Edge.Cuts"))
 (gr_arc (start 87.872576 73.79375) (mid 88.113994 73.223747) (end 88.691314 73.000393) (stroke (width 0.15) (type solid))
  (layer "Edge.Cuts"))
 (gr_line (start 168.230625 74.253126) (end 168.226416 89.237356) (stroke (width 0.15) (type solid)) (layer "Edge.Cuts"))
 (gr_line (start 94.408674 73) (end 93.218046 73) (stroke (width 0.15) (type solid)) (layer "Edge.Cuts"))
 (gr_line (start 179.602501 73.85625) (end 192.785153 73.85625) (stroke (width 0.15) (type solid)) (layer "Edge.Cuts"))
 (gr_line (start 198.502501 73.85625) (end 193.975781 73.85625) (stroke (width 0.15) (type solid)) (layer "Edge.Cuts"))
 (gr_arc (start 85.502501 111.35625) (mid 84.936816 111.121935) (end 84.702501 110.55625) (stroke (width 0.15) (type default))
  (layer "Edge.Cuts"))
 (gr_line (start 118.963202 73.396876) (end 118.967411 88.381106) (stroke (width 0.15) (type solid)) (layer "Edge.Cuts"))
 (segment (start 175.652501 83.148902) (end 178.545153 80.25625) (width 0.2) (layer "B.Cu") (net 1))
 (segment (start 175.652501 87.35625) (end 175.652501 83.148902) (width 0.2) (layer "B.Cu") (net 1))
 (segment (start 175.724501 104.59425) (end 192.307153 104.59425) (width 0.2) (layer "F.Cu") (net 39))
 (segment (start 192.307153 104.59425) (end 193.785153 103.11625) (width 0.2) (layer "F.Cu") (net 39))
 (segment (start 173.602501 106.71625) (end 175.724501 104.59425) (width 0.2) (layer "F.Cu") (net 39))
 (segment (start 192.515153 99.30625) (end 193.785153 98.03625) (width 0.2) (layer "F.Cu") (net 37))
 (segment (start 173.602501 101.63625) (end 175.932501 99.30625) (width 0.2) (layer "F.Cu") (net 37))
 (segment (start 175.932501 99.30625) (end 192.515153 99.30625) (width 0.2) (layer "F.Cu") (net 37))
 (segment (start 175.724501 91.89425) (end 192.307153 91.89425) (width 0.2) (layer "F.Cu") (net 34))
 (segment (start 173.602501 94.01625) (end 175.724501 91.89425) (width 0.2) (layer "F.Cu") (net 34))
 (segment (start 192.307153 91.89425) (end 193.785153 90.41625) (width 0.2) (layer "F.Cu") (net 34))
 (segment (start 173.602501 91.47625) (end 175.772501 89.30625) (width 0.2) (layer "F.Cu") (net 33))
 (segment (start 175.772501 89.30625) (end 192.355153 89.30625) (width 0.2) (layer "F.Cu") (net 33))
 (segment (start 192.355153 89.30625) (end 193.785153 87.87625) (width 0.2) (layer "F.Cu") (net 33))
 (segment (start 173.602501 109.25625) (end 190.185153 109.25625) (width 0.2) (layer "F.Cu") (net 40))
 (segment (start 190.185153 109.25625) (end 193.785153 105.65625) (width 0.2) (layer "F.Cu") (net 40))
 (segment (start 173.602501 104.17625) (end 175.972501 101.80625) (width 0.2) (layer "F.Cu") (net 38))
 (segment (start 192.555153 101.80625) (end 193.785153 100.57625) (width 0.2) (layer "F.Cu") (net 38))
 (segment (start 175.972501 101.80625) (end 192.555153 101.80625) (width 0.2) (layer "F.Cu") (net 38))
 (segment (start 173.602501 99.09625) (end 175.724501 96.97425) (width 0.2) (layer "F.Cu") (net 36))
 (segment (start 175.724501 96.97425) (end 192.307153 96.97425) (width 0.2) (layer "F.Cu") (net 36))
 (segment (start 192.307153 96.97425) (end 193.785153 95.49625) (width 0.2) (layer "F.Cu") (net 36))
 (segment (start 192.307153 94.43425) (end 193.785153 92.95625) (width 0.2) (layer "F.Cu") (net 35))
 (segment (start 173.602501 96.55625) (end 175.724501 94.43425) (width 0.2) (layer "F.Cu") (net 35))
 (segment (start 175.724501 94.43425) (end 192.307153 94.43425) (width 0.2) (layer "F.Cu") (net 35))
 (segment (start 182.563153 96.97425) (end 178.545153 92.95625) (width 0.2) (layer "B.Cu") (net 7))
 (segment (start 199.440501 96.97425) (end 182.563153 96.97425) (width 0.2) (layer "B.Cu") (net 7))
 (segment (start 199.852501 97.38625) (end 199.440501 96.97425) (width 0.2) (layer "B.Cu") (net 7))
 (segment (start 199.852501 107.54625) (end 196.884501 104.57825) (width 0.2) (layer "B.Cu") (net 11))
 (segment (start 196.884501 104.57825) (end 180.007153 104.57825) (width 0.2) (layer "B.Cu") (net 11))
 (segment (start 180.007153 104.57825) (end 178.545153 103.11625) (width 0.2) (layer "B.Cu") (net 11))
 (segment (start 182.147153 104.17825) (end 178.545153 100.57625) (width 0.2) (layer "B.Cu") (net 10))
 (segment (start 199.852501 105.00625) (end 199.024501 104.17825) (width 0.2) (layer "B.Cu") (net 10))
 (segment (start 199.024501 104.17825) (end 182.147153 104.17825) (width 0.2) (layer "B.Cu") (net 10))
 (segment (start 171.052501 86.25625) (end 171.852501 85.45625) (width 0.2) (layer "F.Cu") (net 2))
 (segment (start 171.852501 85.45625) (end 178.425153 85.45625) (width 0.2) (layer "F.Cu") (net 2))
 (segment (start 178.425153 85.45625) (end 178.545153 85.33625) (width 0.2) (layer "F.Cu") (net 2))
 (segment (start 171.052501 79.25625) (end 171.114501 79.19425) (width 0.2) (layer "B.Cu") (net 4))
 (segment (start 192.307153 79.19425) (end 193.785153 77.71625) (width 0.2) (layer "B.Cu") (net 4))
 (segment (start 171.114501 79.19425) (end 192.307153 79.19425) (width 0.2) (layer "B.Cu") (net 4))
 (segment (start 199.440501 102.05425) (end 182.563153 102.05425) (width 0.2) (layer "B.Cu") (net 9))
 (segment (start 182.563153 102.05425) (end 178.545153 98.03625) (width 0.2) (layer "B.Cu") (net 9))
 (segment (start 199.852501 102.46625) (end 199.440501 102.05425) (width 0.2) (layer "B.Cu") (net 9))
 (segment (start 182.563153 94.43425) (end 178.545153 90.41625) (width 0.2) (layer "B.Cu") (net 6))
 (segment (start 199.440501 94.43425) (end 182.563153 94.43425) (width 0.2) (layer "B.Cu") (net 6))
 (segment (start 199.852501 94.84625) (end 199.440501 94.43425) (width 0.2) (layer "B.Cu") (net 6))
 (segment (start 199.852501 110.08625) (end 182.975153 110.08625) (width 0.2) (layer "B.Cu") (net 12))
 (segment (start 182.975153 110.08625) (end 178.545153 105.65625) (width 0.2) (layer "B.Cu") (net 12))
 (segment (start 199.440501 91.89425) (end 182.563153 91.89425) (width 0.2) (layer "B.Cu") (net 5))
 (segment (start 182.563153 91.89425) (end 178.545153 87.87625) (width 0.2) (layer "B.Cu") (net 5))
 (segment (start 199.852501 92.30625) (end 199.440501 91.89425) (width 0.2) (layer "B.Cu") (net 5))
 (segment (start 199.852501 99.92625) (end 199.440501 99.51425) (width 0.2) (layer "B.Cu") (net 8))
 (segment (start 182.563153 99.51425) (end 178.545153 95.49625) (width 0.2) (layer "B.Cu") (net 8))
 (segment (start 199.440501 99.51425) (end 182.563153 99.51425) (width 0.2) (layer "B.Cu") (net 8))
 (segment (start 110.876751 85.682) (end 111.302501 85.25625) (width 0.2) (layer "B.Cu") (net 22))
 (segment (start 93.822 85.682) (end 110.876751 85.682) (width 0.2) (layer "B.Cu") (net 22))
 (segment (start 92.76 84.62) (end 93.822 85.682) (width 0.2) (layer "B.Cu") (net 22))
 (segment (start 109.62 83) (end 108 84.62) (width 0.2) (layer "F.Cu") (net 21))
 (segment (start 114.3 86.3) (end 111 83) (width 0.2) (layer "F.Cu") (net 21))
 (segment (start 111 83) (end 109.62 83) (width 0.2) (layer "F.Cu") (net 21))
 (segment (start 115.3 86.3) (end 114.3 86.3) (width 0.2) (layer "F.Cu") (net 21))
 (segment (start 113.602501 108.28) (end 96.1 108.28) (width 0.2) (layer "B.Cu") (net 32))
 (segment (start 96.1 108.28) (end 92.76 104.94) (width 0.2) (layer "B.Cu") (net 32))
 (segment (start 113.602501 100.66) (end 111.324501 98.382) (width 0.2) (layer "B.Cu") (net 29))
 (segment (start 93.822 98.382) (end 92.76 97.32) (width 0.2) (layer "B.Cu") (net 29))
 (segment (start 111.324501 98.382) (end 93.822 98.382) (width 0.2) (layer "B.Cu") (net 29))
 (segment (start 105.198 106.79625) (end 106.938 105.05625) (width 0.2) (layer "F.Cu") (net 19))
 (segment (start 106.938 103.462) (end 108 102.4) (width 0.2) (layer "F.Cu") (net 19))
 (segment (start 87.102501 106.79625) (end 105.198 106.79625) (width 0.2) (layer "F.Cu") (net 19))
 (segment (start 106.938 105.05625) (end 106.938 103.462) (width 0.2) (layer "F.Cu") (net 19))
 (segment (start 103.981572 103.878428) (end 108 99.86) (width 0.2) (layer "F.Cu") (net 18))
 (segment (start 87.480323 103.878428) (end 103.981572 103.878428) (width 0.2) (layer "F.Cu") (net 18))
 (segment (start 87.102501 104.25625) (end 87.480323 103.878428) (width 0.2) (layer "F.Cu") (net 18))
 (segment (start 94.238 91.178) (end 92.76 89.7) (width 0.2) (layer "B.Cu") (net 26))
 (segment (start 113.602501 93.04) (end 111.740501 91.178) (width 0.2) (layer "B.Cu") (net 26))
 (segment (start 111.740501 91.178) (end 94.238 91.178) (width 0.2) (layer "B.Cu") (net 26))
 (segment (start 109.2 78.2) (end 108 77) (width 0.2) (layer "F.Cu") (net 24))
 (segment (start 110.7 78.2) (end 109.2 78.2) (width 0.2) (layer "F.Cu") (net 24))
 (segment (start 104.10375 91.05625) (end 108 87.16) (width 0.2) (layer "F.Cu") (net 13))
 (segment (start 87.102501 91.55625) (end 87.602501 91.05625) (width 0.2) (layer "F.Cu") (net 13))
 (segment (start 87.602501 91.05625) (end 104.10375 91.05625) (width 0.2) (layer "F.Cu") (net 13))
 (segment (start 113 90.5) (end 111 88.5) (width 0.2) (layer "B.Cu") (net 25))
 (segment (start 94.1 88.5) (end 92.76 87.16) (width 0.2) (layer "B.Cu") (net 25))
 (segment (start 113.602501 90.5) (end 113 90.5) (width 0.2) (layer "B.Cu") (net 25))
 (segment (start 111 88.5) (end 94.1 88.5) (width 0.2) (layer "B.Cu") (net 25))
 (segment (start 87.602501 96.13625) (end 104.10375 96.13625) (width 0.2) (layer "F.Cu") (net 15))
 (segment (start 104.10375 96.13625) (end 108 92.24) (width 0.2) (layer "F.Cu") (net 15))
 (segment (start 87.102501 96.63625) (end 87.602501 96.13625) (width 0.2) (layer "F.Cu") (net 15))
 (segment (start 111.324501 95.842) (end 93.822 95.842) (width 0.2) (layer "B.Cu") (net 28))
 (segment (start 93.822 95.842) (end 92.76 94.78) (width 0.2) (layer "B.Cu") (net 28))
 (segment (start 113.602501 98.12) (end 111.324501 95.842) (width 0.2) (layer "B.Cu") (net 28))
 (segment (start 113.602501 103.2) (end 111.324501 100.922) (width 0.2) (layer "B.Cu") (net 30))
 (segment (start 93.822 100.922) (end 92.76 99.86) (width 0.2) (layer "B.Cu") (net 30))
 (segment (start 111.324501 100.922) (end 93.822 100.922) (width 0.2) (layer "B.Cu") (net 30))
 (segment (start 87.480751 93.718) (end 103.982 93.718) (width 0.2) (layer "F.Cu") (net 14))
 (segment (start 103.982 93.718) (end 108 89.7) (width 0.2) (layer "F.Cu") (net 14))
 (segment (start 87.102501 94.09625) (end 87.480751 93.718) (width 0.2) (layer "F.Cu") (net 14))
 (segment (start 104.10375 101.21625) (end 108 97.32) (width 0.2) (layer "F.Cu") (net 17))
 (segment (start 87.102501 101.71625) (end 87.602501 101.21625) (width 0.2) (layer "F.Cu") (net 17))
 (segment (start 87.602501 101.21625) (end 104.10375 101.21625) (width 0.2) (layer "F.Cu") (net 17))
 (segment (start 103.982 98.798) (end 108 94.78) (width 0.2) (layer "F.Cu") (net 16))
 (segment (start 87.480751 98.798) (end 103.982 98.798) (width 0.2) (layer "F.Cu") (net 16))
 (segment (start 87.102501 99.17625) (end 87.480751 98.798) (width 0.2) (layer "F.Cu") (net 16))
 (segment (start 113.602501 105.74) (end 111.324501 103.462) (width 0.2) (layer "B.Cu") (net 31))
 (segment (start 93.822 103.462) (end 92.76 102.4) (width 0.2) (layer "B.Cu") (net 31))
 (segment (start 111.324501 103.462) (end 93.822 103.462) (width 0.2) (layer "B.Cu") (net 31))
 (segment (start 111.324501 93.302) (end 93.822 93.302) (width 0.2) (layer "B.Cu") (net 27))
 (segment (start 113.602501 95.58) (end 111.324501 93.302) (width 0.2) (layer "B.Cu") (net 27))
 (segment (start 93.822 93.302) (end 92.76 92.24) (width 0.2) (layer "B.Cu") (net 27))
 (segment (start 87.102501 109.33625) (end 103.60375 109.33625) (width 0.2) (layer "F.Cu") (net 20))
 (segment (start 103.60375 109.33625) (end 108 104.94) (width 0.2) (layer "F.Cu") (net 20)))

